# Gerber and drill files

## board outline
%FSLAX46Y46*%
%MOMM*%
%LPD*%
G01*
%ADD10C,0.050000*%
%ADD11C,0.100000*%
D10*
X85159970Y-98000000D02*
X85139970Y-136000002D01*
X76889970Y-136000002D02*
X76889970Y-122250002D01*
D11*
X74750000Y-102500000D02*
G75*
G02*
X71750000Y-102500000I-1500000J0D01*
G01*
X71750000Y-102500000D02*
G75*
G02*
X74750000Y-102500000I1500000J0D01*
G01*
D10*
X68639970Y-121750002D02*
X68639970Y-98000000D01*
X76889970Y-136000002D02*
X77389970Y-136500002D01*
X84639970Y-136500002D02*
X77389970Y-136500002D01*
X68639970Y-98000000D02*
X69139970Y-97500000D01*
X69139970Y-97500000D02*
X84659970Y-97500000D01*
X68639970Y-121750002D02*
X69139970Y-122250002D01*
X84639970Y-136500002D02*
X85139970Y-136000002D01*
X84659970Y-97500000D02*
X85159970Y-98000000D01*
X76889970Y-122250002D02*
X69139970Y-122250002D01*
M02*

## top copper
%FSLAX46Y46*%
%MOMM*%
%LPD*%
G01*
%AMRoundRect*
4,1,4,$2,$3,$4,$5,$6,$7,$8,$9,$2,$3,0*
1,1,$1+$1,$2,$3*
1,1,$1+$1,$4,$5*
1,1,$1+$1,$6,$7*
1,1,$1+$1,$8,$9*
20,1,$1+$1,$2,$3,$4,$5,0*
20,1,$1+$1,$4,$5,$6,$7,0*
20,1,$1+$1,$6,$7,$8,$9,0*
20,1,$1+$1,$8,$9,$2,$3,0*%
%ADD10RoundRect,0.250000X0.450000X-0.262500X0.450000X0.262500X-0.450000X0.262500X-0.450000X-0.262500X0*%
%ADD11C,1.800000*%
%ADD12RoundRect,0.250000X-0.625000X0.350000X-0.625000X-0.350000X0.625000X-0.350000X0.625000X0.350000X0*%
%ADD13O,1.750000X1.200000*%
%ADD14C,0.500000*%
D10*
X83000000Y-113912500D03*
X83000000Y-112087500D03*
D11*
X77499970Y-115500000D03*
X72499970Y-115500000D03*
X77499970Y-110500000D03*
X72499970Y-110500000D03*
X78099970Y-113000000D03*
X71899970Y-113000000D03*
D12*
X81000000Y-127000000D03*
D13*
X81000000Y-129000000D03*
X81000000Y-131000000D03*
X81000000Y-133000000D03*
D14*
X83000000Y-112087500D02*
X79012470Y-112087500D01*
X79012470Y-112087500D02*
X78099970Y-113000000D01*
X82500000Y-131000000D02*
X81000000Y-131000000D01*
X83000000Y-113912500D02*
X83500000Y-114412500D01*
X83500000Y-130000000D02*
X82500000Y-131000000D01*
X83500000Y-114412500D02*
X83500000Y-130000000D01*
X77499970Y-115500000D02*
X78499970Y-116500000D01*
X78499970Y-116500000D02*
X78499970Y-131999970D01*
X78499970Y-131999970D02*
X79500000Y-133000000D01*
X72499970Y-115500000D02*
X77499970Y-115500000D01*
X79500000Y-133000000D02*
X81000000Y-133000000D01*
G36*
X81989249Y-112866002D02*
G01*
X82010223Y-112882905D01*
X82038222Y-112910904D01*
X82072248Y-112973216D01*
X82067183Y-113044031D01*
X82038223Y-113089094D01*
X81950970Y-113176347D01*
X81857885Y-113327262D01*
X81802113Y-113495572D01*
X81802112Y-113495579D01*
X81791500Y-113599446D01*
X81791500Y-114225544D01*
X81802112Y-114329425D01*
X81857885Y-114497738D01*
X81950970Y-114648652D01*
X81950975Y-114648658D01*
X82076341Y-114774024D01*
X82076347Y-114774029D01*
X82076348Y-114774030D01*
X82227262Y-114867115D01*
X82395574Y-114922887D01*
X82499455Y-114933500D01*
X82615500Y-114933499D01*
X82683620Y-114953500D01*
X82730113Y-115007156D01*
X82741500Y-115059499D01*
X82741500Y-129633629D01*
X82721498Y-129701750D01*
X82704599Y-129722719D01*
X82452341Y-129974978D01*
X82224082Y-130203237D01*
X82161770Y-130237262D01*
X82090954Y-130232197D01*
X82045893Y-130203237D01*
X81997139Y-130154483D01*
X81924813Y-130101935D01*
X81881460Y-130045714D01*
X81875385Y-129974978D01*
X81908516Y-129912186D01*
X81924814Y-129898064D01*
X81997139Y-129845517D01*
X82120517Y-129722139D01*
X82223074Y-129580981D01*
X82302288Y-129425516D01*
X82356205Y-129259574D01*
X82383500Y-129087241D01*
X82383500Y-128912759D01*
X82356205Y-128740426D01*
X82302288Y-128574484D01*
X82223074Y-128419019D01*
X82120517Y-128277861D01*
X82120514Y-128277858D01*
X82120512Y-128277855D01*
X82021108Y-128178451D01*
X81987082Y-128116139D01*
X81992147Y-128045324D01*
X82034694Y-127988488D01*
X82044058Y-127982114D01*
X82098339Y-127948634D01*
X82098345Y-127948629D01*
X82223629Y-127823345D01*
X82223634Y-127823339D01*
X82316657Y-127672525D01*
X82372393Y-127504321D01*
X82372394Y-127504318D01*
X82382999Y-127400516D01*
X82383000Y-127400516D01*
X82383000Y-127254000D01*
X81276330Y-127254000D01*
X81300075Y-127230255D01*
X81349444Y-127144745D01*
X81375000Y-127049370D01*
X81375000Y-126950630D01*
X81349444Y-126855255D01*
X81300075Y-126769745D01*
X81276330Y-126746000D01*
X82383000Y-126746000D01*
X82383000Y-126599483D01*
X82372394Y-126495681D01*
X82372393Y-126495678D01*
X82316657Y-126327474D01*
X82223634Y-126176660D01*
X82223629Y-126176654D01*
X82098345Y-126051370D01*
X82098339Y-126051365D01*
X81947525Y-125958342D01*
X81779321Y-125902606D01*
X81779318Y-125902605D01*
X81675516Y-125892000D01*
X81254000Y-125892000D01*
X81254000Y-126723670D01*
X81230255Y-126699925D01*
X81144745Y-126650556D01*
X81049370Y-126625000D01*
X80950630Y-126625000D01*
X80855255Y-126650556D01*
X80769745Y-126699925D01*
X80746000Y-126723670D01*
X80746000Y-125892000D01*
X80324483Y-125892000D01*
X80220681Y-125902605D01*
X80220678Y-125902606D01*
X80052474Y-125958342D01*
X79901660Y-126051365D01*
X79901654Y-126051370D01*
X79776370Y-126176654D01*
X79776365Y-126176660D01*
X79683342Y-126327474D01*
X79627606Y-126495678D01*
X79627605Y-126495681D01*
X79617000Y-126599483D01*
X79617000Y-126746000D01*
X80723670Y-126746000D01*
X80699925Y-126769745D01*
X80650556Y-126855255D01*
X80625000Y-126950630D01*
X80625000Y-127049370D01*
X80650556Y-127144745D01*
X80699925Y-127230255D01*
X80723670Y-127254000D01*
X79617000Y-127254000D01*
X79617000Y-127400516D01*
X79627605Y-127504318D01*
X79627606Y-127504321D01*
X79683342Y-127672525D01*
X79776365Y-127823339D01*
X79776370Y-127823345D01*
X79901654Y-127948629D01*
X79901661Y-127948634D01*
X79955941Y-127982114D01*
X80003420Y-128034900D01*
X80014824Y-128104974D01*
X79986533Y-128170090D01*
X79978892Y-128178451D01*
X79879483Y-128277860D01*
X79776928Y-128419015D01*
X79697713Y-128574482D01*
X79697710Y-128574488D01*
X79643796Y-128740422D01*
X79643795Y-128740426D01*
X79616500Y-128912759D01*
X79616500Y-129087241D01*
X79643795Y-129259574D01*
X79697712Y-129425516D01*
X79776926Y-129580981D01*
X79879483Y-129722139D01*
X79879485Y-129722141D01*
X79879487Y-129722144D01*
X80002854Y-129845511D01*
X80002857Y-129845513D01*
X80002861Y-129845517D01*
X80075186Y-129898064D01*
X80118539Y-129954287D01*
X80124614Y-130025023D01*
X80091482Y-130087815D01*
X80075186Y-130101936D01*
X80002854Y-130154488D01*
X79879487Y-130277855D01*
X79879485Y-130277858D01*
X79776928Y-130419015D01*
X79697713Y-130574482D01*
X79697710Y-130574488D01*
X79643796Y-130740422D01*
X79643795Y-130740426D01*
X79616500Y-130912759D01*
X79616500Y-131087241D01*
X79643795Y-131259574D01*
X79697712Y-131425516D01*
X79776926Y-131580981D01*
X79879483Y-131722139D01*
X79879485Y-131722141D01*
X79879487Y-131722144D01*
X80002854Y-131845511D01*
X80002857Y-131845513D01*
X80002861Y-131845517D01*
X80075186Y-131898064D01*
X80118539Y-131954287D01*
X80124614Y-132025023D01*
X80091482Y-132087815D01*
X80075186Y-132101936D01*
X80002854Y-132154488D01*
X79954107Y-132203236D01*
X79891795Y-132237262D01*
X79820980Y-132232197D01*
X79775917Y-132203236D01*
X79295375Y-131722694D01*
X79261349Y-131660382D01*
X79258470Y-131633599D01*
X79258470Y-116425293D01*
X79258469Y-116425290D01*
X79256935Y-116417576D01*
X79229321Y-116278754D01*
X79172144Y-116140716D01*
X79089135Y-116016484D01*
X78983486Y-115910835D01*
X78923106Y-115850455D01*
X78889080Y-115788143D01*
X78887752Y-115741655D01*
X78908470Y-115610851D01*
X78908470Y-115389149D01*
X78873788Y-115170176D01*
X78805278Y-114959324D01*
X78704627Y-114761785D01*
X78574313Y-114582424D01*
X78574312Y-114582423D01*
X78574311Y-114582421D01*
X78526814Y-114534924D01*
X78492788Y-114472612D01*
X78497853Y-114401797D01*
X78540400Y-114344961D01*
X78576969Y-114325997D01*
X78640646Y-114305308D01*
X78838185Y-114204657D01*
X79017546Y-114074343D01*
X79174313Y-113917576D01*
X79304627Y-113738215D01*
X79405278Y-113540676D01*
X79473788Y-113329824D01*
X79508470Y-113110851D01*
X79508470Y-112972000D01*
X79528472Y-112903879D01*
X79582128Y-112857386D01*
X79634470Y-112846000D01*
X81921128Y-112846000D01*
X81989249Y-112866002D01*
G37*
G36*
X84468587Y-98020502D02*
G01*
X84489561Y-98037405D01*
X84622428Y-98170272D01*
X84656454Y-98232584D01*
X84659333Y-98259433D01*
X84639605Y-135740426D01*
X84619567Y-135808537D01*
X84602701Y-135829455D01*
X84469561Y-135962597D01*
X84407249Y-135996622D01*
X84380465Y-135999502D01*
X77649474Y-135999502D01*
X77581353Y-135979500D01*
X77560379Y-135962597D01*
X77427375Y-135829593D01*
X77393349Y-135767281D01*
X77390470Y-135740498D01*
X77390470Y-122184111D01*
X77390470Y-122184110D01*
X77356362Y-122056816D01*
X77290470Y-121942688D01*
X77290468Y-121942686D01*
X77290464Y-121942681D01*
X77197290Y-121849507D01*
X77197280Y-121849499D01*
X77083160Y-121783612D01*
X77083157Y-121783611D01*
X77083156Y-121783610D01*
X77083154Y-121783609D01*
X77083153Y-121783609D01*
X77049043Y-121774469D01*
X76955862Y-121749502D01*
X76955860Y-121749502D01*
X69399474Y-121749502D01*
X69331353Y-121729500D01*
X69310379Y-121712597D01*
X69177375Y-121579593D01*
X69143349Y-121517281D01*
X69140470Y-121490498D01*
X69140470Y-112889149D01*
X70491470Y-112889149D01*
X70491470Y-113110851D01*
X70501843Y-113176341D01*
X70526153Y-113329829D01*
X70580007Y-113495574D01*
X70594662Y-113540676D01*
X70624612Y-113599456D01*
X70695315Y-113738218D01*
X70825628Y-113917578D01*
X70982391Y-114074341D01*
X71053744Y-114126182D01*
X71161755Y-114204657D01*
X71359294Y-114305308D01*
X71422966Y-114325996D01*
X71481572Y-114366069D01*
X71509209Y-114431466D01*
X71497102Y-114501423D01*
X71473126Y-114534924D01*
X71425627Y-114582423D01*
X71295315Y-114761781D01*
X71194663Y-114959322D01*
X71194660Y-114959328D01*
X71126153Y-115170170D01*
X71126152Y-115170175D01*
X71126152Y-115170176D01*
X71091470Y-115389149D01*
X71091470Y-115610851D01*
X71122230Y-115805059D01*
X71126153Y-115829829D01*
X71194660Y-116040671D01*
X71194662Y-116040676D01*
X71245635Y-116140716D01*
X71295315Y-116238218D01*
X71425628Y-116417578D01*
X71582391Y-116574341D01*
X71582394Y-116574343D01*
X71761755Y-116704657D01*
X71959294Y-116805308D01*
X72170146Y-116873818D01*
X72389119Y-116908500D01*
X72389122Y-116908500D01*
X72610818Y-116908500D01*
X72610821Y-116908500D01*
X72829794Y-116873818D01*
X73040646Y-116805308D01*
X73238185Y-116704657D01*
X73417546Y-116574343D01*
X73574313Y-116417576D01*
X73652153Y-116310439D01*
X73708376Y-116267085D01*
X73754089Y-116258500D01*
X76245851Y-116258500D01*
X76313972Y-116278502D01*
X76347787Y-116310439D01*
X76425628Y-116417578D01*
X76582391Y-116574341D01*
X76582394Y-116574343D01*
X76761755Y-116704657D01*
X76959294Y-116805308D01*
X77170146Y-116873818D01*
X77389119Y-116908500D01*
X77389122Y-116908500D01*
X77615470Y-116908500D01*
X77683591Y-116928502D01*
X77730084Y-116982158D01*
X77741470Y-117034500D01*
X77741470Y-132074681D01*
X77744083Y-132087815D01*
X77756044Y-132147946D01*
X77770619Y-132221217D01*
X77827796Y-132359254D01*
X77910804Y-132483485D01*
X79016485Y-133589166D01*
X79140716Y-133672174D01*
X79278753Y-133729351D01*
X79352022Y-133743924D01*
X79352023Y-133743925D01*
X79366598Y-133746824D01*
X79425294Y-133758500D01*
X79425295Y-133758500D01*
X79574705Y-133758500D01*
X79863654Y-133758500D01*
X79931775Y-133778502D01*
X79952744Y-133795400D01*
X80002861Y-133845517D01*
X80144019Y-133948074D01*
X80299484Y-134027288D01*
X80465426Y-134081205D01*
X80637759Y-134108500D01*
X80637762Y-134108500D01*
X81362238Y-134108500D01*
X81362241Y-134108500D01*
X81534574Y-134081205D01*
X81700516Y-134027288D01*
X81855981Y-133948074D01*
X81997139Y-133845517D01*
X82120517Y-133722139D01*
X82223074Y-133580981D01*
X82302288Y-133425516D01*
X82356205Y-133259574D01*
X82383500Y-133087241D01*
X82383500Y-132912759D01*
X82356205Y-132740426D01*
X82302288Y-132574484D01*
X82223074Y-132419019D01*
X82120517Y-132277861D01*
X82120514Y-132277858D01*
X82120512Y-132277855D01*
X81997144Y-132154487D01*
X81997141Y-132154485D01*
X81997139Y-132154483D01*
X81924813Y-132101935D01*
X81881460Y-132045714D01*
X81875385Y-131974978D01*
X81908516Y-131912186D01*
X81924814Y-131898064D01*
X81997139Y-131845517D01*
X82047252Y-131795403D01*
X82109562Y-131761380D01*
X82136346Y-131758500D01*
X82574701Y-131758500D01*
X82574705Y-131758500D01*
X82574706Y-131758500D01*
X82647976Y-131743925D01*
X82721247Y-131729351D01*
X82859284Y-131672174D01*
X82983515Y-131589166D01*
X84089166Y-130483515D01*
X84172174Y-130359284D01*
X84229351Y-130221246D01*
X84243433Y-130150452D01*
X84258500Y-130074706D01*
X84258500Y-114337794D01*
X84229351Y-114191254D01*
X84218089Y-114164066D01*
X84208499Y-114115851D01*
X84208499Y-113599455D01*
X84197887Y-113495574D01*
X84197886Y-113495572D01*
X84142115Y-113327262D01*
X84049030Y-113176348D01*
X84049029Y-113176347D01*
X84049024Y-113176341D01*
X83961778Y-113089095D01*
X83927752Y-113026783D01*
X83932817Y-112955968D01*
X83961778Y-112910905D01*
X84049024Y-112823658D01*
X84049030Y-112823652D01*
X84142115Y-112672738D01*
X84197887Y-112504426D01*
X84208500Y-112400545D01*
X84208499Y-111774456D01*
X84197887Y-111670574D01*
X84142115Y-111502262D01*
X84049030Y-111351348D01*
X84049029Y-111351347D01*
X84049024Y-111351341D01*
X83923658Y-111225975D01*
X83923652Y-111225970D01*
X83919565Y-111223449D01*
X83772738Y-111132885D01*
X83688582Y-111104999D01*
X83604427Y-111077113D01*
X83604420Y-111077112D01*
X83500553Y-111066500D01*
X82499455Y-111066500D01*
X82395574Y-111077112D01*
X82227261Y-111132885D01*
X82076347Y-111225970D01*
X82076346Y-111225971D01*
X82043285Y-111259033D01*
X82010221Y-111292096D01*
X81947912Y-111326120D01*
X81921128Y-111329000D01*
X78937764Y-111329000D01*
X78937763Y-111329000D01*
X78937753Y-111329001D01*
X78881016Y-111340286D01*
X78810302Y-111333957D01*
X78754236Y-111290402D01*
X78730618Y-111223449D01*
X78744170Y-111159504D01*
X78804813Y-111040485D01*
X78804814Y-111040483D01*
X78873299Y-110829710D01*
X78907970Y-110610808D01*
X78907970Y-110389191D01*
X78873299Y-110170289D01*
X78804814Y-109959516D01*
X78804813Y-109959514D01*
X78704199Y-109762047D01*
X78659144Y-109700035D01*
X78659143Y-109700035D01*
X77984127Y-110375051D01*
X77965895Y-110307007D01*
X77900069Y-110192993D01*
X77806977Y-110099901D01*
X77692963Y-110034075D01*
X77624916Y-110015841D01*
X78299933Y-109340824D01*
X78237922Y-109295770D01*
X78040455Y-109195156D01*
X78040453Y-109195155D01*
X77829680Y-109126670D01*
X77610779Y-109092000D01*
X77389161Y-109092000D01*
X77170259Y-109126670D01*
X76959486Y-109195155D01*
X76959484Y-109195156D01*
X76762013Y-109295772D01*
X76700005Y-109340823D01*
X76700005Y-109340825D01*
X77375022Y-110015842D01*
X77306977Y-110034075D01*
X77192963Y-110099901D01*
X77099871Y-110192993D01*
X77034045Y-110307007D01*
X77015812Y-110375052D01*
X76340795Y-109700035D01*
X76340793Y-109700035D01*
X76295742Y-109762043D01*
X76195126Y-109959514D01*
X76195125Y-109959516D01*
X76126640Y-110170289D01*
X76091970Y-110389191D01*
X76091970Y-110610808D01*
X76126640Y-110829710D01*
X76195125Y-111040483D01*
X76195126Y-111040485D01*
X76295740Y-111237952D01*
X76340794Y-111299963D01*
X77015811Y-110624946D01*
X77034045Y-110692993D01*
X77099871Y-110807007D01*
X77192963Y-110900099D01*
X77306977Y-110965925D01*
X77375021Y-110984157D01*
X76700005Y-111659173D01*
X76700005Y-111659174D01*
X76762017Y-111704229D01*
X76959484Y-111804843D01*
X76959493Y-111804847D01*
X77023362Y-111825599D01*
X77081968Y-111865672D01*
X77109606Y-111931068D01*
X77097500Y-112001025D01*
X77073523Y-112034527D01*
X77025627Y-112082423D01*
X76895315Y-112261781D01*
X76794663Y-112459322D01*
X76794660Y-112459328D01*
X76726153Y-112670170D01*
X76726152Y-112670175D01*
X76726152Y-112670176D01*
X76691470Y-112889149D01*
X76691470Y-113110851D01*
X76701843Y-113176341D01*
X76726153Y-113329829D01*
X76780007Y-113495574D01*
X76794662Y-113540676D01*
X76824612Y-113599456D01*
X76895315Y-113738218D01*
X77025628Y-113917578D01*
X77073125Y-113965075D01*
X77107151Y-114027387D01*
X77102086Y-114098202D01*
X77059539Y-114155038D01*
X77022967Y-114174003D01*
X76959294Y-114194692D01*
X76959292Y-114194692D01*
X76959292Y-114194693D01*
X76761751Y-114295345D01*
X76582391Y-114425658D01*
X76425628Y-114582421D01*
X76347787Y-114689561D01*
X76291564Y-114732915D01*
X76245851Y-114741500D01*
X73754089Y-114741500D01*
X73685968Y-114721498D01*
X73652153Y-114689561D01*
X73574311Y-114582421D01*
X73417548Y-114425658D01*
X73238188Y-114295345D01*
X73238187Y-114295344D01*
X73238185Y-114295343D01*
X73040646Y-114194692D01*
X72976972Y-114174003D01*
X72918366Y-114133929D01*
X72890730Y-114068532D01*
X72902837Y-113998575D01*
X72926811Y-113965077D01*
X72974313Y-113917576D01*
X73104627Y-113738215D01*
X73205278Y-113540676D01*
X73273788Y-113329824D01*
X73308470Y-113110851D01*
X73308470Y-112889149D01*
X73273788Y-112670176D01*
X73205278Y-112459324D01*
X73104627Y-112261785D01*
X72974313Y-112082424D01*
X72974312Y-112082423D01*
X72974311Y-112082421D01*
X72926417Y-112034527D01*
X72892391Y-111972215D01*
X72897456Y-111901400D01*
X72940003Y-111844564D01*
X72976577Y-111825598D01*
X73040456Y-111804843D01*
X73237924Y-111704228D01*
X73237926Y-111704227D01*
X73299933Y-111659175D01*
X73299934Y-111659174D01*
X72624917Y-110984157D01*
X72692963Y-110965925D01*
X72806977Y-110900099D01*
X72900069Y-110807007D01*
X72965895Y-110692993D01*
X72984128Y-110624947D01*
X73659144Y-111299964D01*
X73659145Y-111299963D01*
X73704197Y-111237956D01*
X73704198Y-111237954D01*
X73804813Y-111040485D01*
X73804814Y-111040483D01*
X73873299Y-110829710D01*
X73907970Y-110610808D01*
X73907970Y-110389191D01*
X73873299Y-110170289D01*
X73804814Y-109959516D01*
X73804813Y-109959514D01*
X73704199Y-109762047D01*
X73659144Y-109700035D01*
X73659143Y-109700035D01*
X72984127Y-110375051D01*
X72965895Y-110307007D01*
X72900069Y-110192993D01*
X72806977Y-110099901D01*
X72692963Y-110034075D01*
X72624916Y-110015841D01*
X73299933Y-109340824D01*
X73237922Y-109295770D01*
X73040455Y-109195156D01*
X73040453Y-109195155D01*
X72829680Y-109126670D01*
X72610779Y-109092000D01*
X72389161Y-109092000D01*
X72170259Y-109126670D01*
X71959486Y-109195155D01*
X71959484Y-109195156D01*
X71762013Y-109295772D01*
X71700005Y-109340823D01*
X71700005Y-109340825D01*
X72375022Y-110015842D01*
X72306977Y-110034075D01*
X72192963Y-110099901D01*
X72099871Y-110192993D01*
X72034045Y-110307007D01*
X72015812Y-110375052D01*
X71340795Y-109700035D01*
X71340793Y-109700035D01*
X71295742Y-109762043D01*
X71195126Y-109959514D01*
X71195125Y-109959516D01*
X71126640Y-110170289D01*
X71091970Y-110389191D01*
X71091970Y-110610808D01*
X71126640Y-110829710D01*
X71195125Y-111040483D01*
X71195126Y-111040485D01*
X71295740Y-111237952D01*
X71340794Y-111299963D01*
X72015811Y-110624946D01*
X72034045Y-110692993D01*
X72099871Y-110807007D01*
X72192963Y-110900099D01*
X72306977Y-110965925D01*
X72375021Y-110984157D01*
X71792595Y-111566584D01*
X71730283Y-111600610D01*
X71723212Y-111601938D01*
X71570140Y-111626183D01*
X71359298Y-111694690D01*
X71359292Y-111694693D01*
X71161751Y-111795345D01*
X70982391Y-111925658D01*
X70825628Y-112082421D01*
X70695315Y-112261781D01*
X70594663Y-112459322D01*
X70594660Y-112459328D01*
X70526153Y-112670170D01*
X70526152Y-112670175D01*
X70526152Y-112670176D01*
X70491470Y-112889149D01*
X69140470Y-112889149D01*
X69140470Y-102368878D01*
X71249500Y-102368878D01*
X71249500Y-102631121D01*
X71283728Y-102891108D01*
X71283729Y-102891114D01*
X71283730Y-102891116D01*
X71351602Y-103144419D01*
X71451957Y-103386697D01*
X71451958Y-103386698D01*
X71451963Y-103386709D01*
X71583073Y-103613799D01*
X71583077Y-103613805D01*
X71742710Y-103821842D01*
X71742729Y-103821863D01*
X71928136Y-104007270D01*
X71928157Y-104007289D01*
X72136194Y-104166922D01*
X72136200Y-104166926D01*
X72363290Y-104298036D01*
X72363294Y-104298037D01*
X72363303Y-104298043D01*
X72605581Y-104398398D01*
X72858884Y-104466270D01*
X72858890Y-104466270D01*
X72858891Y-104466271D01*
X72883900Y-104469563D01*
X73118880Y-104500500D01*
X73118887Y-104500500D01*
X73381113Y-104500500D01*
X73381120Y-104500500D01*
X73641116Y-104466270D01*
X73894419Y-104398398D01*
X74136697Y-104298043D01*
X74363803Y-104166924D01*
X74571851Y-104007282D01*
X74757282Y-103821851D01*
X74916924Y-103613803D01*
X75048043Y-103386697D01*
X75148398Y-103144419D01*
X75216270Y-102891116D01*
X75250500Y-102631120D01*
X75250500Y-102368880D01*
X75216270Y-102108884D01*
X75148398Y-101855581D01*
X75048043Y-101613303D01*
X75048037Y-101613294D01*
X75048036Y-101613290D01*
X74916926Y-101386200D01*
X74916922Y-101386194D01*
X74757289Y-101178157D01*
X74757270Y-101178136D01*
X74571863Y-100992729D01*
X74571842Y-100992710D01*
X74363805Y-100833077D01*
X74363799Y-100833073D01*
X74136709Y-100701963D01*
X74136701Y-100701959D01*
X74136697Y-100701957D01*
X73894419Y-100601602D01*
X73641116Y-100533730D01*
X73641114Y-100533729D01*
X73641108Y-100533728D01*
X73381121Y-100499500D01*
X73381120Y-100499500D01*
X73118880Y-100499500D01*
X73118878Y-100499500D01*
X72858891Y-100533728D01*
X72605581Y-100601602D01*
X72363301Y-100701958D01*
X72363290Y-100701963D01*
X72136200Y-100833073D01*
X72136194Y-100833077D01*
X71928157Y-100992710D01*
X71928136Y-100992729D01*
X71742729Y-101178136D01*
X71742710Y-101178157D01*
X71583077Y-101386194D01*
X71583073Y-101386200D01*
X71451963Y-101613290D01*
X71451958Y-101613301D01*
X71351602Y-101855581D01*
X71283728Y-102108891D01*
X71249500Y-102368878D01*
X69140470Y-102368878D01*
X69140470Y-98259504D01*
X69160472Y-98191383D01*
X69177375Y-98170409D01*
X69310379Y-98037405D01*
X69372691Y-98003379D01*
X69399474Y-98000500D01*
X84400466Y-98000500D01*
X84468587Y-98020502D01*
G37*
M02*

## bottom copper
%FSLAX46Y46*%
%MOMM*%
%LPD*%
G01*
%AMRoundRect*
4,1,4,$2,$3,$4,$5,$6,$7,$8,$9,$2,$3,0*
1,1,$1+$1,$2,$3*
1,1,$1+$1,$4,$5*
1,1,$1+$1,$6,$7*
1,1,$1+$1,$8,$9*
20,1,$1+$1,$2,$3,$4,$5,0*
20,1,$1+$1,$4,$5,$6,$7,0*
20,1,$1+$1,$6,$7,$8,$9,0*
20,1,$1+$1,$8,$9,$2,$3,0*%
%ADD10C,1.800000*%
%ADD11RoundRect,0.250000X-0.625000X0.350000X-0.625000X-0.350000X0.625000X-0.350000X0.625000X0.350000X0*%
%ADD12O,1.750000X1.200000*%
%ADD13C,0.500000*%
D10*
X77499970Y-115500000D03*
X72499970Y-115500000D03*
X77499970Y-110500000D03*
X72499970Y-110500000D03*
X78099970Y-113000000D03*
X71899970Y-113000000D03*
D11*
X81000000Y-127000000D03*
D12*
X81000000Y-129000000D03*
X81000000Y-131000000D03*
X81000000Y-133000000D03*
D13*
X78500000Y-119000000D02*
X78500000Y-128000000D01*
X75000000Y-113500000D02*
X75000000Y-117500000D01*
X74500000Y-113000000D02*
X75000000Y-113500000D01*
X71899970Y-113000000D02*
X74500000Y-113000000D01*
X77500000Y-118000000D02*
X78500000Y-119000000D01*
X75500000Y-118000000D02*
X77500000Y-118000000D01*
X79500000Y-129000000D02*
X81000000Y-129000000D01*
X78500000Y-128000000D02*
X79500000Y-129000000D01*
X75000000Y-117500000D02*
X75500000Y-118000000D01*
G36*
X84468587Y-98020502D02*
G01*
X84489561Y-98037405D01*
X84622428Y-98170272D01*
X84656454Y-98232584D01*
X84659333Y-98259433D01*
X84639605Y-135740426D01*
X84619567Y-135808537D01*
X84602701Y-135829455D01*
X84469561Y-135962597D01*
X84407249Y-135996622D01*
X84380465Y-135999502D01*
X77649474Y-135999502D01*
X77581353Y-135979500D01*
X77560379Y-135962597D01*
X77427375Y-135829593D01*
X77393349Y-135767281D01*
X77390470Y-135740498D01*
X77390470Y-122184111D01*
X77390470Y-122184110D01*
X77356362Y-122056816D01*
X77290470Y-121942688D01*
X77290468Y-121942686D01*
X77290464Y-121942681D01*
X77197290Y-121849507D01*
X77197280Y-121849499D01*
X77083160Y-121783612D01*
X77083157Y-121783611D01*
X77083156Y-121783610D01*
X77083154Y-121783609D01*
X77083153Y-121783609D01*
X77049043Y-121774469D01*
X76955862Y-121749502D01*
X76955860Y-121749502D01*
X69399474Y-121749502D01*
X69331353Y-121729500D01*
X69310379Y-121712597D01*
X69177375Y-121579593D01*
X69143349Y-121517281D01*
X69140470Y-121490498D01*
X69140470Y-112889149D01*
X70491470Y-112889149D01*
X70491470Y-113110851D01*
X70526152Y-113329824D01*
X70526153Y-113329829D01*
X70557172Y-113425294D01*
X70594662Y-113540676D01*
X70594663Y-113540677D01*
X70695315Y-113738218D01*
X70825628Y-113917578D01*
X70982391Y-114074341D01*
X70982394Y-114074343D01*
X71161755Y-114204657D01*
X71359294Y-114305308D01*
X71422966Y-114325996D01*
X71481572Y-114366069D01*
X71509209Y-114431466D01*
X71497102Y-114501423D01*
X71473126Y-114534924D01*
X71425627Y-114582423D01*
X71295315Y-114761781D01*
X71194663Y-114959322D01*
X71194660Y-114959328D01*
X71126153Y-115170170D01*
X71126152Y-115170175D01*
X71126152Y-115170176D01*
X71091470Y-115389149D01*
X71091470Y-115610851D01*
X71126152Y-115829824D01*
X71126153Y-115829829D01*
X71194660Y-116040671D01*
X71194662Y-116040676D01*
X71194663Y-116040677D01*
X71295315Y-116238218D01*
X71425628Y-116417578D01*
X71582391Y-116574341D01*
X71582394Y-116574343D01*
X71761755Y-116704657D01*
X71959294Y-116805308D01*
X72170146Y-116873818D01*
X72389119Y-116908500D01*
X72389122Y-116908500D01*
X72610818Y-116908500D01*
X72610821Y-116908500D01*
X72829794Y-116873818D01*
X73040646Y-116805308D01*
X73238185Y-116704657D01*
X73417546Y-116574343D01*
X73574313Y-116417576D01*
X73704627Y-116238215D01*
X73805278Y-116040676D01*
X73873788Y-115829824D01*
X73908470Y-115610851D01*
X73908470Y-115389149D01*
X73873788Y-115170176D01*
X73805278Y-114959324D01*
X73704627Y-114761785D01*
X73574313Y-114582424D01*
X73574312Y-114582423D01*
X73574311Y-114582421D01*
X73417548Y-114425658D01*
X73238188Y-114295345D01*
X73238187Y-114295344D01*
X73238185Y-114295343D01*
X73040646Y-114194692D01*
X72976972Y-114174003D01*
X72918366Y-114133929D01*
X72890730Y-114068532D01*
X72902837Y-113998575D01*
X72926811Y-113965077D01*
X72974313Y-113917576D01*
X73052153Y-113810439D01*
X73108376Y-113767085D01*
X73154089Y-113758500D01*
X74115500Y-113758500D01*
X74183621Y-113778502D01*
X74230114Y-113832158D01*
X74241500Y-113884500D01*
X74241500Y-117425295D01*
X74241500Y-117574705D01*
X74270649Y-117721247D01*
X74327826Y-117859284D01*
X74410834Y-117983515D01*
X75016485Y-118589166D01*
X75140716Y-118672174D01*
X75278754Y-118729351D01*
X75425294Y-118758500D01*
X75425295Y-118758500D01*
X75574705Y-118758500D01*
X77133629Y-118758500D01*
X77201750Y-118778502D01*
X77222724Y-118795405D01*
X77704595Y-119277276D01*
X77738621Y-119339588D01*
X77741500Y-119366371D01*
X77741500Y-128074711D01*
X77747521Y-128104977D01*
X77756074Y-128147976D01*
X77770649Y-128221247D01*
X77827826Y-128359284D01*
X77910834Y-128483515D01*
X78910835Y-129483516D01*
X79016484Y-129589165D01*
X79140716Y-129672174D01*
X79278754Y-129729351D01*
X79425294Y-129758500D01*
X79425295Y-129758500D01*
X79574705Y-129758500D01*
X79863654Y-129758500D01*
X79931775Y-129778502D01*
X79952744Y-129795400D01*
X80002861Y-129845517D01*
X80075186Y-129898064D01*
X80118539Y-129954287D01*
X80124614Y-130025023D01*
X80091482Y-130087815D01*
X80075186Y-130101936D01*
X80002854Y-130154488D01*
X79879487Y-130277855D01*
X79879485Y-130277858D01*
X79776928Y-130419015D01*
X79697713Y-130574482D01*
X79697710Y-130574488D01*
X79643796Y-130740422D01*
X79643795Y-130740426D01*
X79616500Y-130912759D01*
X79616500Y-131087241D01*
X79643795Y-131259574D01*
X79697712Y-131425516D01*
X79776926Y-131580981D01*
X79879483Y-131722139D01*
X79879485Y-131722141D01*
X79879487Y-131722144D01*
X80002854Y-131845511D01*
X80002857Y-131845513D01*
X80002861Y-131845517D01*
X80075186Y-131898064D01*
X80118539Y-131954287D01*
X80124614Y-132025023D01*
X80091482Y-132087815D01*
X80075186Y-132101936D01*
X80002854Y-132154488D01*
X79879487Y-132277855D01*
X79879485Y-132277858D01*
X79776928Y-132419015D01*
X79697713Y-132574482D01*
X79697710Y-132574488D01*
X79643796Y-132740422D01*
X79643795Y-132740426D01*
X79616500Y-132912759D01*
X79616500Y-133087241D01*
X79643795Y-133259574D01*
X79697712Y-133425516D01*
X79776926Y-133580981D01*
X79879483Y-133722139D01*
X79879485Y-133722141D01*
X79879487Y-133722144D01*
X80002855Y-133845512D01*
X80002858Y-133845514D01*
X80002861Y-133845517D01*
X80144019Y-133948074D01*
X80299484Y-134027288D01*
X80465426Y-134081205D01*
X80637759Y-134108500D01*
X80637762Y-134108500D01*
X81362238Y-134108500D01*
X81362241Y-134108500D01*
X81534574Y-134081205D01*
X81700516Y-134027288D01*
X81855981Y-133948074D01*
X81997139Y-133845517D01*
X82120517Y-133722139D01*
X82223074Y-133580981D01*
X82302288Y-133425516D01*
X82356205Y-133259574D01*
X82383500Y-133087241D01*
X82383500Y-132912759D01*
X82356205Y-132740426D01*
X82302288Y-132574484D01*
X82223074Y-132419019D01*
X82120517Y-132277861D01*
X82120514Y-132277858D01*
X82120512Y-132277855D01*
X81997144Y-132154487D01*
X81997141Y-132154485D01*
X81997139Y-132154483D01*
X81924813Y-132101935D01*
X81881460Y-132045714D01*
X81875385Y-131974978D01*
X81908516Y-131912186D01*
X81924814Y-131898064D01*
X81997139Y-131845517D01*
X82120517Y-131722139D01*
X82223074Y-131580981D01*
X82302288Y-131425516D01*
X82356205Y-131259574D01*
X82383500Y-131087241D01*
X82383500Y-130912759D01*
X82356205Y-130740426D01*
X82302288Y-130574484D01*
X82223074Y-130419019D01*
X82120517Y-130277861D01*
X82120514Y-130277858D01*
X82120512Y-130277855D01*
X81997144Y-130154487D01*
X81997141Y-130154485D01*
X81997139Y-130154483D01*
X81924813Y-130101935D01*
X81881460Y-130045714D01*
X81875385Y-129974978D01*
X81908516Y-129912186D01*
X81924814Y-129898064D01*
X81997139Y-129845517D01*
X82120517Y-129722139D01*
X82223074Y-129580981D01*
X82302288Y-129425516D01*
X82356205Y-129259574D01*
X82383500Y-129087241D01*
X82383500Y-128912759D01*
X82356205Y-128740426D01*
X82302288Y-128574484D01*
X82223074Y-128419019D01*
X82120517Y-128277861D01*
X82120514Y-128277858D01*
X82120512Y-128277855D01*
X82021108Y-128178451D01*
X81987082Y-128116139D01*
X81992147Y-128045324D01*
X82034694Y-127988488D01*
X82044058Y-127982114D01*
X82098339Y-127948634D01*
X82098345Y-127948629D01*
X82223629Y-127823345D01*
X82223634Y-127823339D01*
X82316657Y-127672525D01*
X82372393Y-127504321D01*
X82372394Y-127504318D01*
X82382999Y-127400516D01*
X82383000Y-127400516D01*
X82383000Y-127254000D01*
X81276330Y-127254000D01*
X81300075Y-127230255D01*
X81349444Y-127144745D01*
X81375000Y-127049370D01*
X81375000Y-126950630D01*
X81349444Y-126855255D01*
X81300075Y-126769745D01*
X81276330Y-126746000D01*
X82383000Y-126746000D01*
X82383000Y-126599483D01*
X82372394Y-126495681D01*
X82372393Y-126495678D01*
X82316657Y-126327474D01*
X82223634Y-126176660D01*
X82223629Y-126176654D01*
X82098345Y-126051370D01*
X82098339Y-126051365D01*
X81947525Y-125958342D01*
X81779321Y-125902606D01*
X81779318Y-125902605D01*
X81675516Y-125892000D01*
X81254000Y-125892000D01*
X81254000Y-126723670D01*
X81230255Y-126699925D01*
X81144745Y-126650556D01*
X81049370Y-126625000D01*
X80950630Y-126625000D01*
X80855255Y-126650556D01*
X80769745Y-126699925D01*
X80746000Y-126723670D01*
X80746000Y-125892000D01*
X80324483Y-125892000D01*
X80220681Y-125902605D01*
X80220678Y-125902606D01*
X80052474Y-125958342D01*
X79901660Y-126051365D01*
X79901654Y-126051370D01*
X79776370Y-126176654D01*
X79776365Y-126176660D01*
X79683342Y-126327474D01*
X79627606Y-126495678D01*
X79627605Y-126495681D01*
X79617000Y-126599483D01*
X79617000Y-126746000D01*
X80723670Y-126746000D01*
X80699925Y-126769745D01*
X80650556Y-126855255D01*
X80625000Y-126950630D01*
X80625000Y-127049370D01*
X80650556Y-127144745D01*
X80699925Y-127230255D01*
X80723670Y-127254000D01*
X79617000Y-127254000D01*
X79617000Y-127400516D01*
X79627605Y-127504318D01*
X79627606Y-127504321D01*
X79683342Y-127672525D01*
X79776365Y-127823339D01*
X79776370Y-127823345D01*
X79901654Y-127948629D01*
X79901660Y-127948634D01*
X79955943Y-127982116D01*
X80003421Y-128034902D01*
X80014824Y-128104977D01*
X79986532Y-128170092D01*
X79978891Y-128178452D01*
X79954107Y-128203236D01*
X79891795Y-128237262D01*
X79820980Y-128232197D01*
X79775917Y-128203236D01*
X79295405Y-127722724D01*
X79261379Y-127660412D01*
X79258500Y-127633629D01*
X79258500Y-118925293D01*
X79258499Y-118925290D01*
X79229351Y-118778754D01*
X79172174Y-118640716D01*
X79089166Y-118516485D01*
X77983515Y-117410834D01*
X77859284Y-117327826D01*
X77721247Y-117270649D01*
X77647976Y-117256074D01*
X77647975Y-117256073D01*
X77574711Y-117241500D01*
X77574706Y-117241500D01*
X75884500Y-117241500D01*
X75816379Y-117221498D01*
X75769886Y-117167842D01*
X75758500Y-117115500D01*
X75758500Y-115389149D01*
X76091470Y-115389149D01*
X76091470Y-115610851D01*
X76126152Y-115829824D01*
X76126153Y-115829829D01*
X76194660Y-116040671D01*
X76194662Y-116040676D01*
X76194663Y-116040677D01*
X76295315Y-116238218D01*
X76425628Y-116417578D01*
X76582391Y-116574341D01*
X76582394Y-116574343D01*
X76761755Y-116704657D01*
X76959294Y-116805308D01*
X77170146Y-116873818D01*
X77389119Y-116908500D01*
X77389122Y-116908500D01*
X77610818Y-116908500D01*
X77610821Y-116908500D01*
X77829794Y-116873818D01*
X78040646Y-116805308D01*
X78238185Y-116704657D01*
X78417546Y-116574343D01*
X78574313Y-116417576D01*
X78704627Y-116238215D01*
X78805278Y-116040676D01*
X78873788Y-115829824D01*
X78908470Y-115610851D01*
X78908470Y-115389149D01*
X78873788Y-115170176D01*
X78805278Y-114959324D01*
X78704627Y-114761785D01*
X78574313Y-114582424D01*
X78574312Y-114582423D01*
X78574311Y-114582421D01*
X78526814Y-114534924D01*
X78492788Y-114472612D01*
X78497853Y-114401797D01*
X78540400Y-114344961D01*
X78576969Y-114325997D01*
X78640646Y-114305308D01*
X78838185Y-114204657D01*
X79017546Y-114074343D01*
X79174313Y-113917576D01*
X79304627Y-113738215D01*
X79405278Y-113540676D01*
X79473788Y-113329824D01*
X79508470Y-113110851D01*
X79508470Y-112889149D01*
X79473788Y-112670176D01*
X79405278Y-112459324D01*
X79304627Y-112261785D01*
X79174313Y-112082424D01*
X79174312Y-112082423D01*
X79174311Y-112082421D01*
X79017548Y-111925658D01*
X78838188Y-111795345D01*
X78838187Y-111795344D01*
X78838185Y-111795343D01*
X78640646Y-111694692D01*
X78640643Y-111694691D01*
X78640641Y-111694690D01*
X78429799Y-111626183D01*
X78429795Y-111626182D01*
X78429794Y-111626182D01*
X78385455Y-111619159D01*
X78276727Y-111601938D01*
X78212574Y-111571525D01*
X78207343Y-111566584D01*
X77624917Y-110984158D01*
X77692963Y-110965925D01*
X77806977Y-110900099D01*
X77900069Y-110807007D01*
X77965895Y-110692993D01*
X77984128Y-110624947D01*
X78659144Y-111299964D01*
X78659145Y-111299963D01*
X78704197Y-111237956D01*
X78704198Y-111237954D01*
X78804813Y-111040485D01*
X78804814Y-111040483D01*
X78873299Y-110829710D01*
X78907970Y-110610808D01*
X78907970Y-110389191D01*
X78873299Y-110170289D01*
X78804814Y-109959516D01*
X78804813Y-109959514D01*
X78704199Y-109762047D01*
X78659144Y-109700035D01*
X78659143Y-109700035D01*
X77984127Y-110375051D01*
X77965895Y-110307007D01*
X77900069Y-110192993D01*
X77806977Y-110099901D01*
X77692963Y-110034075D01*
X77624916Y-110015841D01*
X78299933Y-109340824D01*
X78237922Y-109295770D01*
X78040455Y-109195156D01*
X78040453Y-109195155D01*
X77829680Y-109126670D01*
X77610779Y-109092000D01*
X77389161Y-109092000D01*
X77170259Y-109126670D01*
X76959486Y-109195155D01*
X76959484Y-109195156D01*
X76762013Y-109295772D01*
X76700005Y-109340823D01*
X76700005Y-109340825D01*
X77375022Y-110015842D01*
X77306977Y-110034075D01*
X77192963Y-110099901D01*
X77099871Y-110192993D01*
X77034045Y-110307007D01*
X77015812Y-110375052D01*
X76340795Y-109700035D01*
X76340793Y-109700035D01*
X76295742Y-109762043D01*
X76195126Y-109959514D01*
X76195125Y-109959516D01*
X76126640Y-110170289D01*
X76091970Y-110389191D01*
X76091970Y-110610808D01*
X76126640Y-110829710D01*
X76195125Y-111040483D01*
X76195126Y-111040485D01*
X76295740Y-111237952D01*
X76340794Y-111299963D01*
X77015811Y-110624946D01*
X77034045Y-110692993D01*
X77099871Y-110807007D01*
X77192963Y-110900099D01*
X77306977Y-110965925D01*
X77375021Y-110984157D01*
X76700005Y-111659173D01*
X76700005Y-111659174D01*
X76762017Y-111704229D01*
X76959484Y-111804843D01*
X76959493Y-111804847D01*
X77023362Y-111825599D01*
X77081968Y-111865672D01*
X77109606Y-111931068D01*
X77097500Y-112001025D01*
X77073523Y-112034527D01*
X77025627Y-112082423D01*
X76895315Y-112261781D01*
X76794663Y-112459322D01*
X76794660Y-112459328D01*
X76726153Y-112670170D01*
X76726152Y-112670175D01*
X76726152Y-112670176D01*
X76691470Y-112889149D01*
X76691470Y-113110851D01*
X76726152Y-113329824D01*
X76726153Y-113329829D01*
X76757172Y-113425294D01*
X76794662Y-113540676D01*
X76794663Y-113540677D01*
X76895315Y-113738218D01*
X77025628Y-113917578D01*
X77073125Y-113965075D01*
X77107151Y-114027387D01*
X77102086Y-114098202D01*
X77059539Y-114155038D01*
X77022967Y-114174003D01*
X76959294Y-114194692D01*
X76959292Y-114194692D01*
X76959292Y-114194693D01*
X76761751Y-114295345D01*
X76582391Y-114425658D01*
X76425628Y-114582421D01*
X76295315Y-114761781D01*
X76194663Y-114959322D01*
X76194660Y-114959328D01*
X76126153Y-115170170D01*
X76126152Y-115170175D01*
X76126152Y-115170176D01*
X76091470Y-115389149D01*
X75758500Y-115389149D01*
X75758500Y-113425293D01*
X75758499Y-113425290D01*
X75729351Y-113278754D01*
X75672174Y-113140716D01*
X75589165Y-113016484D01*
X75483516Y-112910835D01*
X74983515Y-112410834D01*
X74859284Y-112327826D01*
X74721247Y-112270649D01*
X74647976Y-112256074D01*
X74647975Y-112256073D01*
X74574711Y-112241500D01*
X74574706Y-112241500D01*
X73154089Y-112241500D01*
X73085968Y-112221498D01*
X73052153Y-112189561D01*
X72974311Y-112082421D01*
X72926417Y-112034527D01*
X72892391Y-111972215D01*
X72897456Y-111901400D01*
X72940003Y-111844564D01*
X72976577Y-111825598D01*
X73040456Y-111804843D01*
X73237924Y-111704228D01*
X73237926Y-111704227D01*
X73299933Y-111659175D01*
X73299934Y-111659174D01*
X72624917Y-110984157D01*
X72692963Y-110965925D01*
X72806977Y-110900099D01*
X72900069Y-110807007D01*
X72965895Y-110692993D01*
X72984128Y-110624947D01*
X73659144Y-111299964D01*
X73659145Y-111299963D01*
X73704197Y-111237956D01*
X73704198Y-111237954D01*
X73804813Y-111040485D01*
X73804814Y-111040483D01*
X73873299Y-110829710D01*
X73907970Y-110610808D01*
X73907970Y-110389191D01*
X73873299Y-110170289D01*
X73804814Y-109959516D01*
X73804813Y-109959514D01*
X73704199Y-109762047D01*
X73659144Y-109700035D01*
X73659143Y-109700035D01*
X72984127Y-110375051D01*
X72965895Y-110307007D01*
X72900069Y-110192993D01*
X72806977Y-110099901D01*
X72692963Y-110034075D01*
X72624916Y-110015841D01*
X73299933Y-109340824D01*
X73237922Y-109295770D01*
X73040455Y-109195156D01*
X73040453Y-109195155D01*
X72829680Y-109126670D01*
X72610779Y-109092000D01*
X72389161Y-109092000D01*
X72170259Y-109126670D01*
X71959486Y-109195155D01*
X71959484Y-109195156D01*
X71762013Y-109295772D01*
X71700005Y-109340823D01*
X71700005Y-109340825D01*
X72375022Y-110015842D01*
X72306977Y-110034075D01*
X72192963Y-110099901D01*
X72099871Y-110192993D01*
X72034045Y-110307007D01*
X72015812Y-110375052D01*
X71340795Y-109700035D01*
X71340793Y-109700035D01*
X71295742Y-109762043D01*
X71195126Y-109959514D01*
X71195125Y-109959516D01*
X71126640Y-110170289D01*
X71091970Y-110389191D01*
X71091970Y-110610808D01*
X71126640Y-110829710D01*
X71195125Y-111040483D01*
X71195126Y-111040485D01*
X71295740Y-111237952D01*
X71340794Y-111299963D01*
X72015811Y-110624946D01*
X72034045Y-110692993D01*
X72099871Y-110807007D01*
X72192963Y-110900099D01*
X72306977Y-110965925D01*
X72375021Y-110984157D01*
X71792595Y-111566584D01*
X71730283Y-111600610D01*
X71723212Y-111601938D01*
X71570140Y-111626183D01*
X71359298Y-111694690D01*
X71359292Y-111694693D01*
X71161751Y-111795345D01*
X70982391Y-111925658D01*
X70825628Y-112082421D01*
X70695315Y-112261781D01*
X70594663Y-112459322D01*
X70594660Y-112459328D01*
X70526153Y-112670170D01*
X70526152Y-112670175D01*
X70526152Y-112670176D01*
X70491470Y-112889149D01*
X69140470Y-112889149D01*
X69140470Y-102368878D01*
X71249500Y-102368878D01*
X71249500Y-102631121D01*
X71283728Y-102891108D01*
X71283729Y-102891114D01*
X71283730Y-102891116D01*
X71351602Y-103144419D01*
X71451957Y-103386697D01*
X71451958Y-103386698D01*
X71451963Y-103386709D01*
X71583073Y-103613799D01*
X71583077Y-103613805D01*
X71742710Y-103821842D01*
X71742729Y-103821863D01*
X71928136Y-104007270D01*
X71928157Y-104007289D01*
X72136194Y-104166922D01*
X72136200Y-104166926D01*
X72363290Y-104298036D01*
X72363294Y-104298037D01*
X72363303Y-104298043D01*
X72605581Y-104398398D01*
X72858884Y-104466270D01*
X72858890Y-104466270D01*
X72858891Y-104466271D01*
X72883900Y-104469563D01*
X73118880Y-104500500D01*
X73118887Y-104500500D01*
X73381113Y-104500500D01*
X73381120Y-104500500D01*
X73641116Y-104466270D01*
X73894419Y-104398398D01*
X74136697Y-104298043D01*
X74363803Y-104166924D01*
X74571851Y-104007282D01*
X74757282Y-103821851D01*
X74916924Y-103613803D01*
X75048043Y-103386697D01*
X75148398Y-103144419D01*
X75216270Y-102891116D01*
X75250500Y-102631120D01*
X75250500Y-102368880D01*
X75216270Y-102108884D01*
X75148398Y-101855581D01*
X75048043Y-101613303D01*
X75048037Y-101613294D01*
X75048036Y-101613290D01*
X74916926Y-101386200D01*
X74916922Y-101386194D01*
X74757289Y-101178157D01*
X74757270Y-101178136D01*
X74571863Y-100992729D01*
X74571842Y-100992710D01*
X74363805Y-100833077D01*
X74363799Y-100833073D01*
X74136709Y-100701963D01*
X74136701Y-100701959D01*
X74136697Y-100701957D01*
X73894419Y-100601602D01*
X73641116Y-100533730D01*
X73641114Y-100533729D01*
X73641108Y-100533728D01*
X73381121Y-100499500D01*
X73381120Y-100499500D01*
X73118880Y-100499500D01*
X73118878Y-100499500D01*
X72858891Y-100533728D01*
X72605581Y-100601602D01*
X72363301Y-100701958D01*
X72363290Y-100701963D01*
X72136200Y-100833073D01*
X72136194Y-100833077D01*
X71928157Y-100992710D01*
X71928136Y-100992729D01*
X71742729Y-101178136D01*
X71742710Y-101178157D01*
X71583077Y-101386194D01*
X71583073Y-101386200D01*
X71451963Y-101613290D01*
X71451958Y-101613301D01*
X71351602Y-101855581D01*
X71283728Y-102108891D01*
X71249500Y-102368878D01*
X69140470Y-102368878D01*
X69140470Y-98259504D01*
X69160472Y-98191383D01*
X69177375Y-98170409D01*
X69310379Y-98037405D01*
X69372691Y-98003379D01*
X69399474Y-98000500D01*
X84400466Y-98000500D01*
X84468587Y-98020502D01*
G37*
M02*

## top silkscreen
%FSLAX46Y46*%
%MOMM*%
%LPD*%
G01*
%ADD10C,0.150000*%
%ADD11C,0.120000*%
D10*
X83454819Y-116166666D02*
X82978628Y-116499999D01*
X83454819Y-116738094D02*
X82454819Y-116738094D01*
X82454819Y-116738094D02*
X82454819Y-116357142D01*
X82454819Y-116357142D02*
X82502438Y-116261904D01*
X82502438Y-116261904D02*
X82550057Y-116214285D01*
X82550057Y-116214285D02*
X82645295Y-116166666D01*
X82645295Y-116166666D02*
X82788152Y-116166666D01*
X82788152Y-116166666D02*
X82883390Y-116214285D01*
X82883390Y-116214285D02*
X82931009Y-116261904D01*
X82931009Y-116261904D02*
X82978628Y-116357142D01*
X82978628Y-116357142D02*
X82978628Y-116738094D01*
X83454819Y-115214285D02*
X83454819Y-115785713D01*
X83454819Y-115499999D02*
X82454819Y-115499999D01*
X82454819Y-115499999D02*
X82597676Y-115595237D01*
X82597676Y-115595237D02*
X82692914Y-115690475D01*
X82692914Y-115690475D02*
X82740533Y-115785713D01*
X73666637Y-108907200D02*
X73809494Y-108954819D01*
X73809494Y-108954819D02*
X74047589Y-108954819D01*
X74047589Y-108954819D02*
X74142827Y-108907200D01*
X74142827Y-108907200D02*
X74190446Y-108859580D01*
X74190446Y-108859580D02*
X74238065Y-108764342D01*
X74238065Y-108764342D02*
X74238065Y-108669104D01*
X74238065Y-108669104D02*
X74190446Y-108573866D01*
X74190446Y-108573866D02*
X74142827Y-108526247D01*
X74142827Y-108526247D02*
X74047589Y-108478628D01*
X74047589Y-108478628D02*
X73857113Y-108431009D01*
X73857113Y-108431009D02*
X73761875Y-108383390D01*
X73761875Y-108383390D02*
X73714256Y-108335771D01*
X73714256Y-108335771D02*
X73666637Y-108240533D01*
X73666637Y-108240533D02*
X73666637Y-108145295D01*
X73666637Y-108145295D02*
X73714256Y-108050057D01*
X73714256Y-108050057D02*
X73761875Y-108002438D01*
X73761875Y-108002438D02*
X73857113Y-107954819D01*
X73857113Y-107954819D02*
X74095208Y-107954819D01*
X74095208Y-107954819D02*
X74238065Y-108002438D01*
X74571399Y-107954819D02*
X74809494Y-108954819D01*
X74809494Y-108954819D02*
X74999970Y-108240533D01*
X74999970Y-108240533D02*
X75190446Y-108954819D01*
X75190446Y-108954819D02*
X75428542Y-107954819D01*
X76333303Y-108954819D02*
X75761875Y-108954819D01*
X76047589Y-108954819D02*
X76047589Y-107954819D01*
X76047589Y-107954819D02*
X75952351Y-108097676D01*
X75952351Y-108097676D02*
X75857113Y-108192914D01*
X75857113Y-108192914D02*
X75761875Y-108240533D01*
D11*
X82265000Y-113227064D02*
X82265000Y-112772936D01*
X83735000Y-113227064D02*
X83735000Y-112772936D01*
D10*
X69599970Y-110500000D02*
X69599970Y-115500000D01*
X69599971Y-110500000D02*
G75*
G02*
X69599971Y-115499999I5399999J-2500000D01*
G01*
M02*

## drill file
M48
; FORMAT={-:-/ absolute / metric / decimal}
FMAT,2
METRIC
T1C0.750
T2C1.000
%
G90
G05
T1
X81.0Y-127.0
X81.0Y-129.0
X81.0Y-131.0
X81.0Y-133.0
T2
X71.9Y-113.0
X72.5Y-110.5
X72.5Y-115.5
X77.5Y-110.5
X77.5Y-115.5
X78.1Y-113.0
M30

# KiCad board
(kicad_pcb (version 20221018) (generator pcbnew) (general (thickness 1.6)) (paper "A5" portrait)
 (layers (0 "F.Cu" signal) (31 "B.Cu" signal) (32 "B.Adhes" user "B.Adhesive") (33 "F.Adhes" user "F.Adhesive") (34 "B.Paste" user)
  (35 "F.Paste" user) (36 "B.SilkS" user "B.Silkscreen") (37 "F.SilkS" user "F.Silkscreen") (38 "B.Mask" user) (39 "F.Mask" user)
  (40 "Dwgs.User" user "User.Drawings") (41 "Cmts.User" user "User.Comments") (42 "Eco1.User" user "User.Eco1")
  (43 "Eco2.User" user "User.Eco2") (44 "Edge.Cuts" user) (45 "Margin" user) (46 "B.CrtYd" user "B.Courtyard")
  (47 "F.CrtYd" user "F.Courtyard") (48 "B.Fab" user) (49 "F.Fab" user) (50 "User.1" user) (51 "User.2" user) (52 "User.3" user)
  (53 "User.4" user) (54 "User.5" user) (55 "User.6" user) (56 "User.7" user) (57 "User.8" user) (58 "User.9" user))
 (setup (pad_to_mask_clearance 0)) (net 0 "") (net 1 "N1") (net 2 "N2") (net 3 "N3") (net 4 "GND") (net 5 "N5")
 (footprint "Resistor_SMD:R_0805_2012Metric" (layer "F.Cu") (at 83 113 90)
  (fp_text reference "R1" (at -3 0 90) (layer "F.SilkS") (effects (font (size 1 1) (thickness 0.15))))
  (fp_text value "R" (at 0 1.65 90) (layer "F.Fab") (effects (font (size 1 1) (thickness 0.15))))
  (fp_line (start -0.227064 -0.735) (end 0.227064 -0.735) (stroke (width 0.12) (type solid)) (layer "F.SilkS"))
  (fp_line (start -0.227064 0.735) (end 0.227064 0.735) (stroke (width 0.12) (type solid)) (layer "F.SilkS"))
  (pad "1" smd roundrect (at -0.9125 0 90) (size 1.025 1.4) (layers "F.Cu" "F.Paste" "F.Mask") (roundrect_rratio 0.243902439) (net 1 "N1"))
  (pad "2" smd roundrect (at 0.9125 0 90) (size 1.025 1.4) (layers "F.Cu" "F.Paste" "F.Mask") (roundrect_rratio 0.243902439) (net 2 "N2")))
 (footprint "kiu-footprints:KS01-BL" (layer "F.Cu") (at 74.99997 113 180)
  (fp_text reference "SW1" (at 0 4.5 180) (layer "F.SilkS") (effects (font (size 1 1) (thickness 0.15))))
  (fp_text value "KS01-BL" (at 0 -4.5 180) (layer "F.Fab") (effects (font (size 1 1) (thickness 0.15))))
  (fp_line (start 5.4 2.5) (end 5.4 -2.5) (stroke (width 0.15) (type solid)) (layer "F.SilkS"))
  (fp_arc (start 5.399999 2.5) (mid -5.950629 0) (end 5.399999 -2.499999) (stroke (width 0.15) (type solid)) (layer "F.SilkS"))
  (pad "1" thru_hole circle (at -2.5 -2.5 180) (size 1.8 1.8) (drill 1) (layers "*.Cu" "*.Mask") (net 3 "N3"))
  (pad "1" thru_hole circle (at 2.5 -2.5 180) (size 1.8 1.8) (drill 1) (layers "*.Cu" "*.Mask") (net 3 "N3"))
  (pad "2" thru_hole circle (at -2.5 2.5 180) (size 1.8 1.8) (drill 1) (layers "*.Cu" "*.Mask") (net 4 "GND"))
  (pad "2" thru_hole circle (at 2.5 2.5 180) (size 1.8 1.8) (drill 1) (layers "*.Cu" "*.Mask") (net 4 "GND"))
  (pad "5" thru_hole circle (at -3.1 0 180) (size 1.8 1.8) (drill 1) (layers "*.Cu" "*.Mask") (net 2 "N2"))
  (pad "6" thru_hole circle (at 3.1 0 180) (size 1.8 1.8) (drill 1) (layers "*.Cu" "*.Mask") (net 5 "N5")))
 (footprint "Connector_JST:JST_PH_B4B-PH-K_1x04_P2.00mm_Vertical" (layer "B.Cu") (at 81 127 -90)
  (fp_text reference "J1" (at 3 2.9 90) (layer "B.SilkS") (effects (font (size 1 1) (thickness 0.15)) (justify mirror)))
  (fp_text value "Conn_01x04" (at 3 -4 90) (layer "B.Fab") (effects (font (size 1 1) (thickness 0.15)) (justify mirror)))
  (pad "1" thru_hole roundrect (at 0 0 270) (size 1.2 1.75) (drill 0.75) (layers "*.Cu" "*.Mask") (roundrect_rratio 0.2083333333)
   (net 4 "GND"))
  (pad "2" thru_hole oval (at 2 0 270) (size 1.2 1.75) (drill 0.75) (layers "*.Cu" "*.Mask") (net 5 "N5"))
  (pad "3" thru_hole oval (at 4 0 270) (size 1.2 1.75) (drill 0.75) (layers "*.Cu" "*.Mask") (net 1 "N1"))
  (pad "4" thru_hole oval (at 6 0 270) (size 1.2 1.75) (drill 0.75) (layers "*.Cu" "*.Mask") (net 3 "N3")))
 (gr_line (start 85.15997 98) (end 85.13997 136.000002) (stroke (width 0.05) (type solid)) (layer "Edge.Cuts"))
 (gr_line (start 76.88997 136.000002) (end 76.88997 122.250002) (stroke (width 0.05) (type default)) (layer "Edge.Cuts"))
 (gr_circle (center 73.25 102.5) (end 74.75 102.5) (stroke (width 0.1) (type default)) (fill none) (layer "Edge.Cuts"))
 (gr_line (start 68.63997 121.750002) (end 68.63997 98) (stroke (width 0.05) (type default)) (layer "Edge.Cuts"))
 (gr_line (start 76.88997 136.000002) (end 77.38997 136.500002) (stroke (width 0.05) (type default)) (layer "Edge.Cuts"))
 (gr_line (start 84.63997 136.500002) (end 77.38997 136.500002) (stroke (width 0.05) (type solid)) (layer "Edge.Cuts"))
 (gr_line (start 68.63997 98) (end 69.13997 97.5) (stroke (width 0.05) (type default)) (layer "Edge.Cuts"))
 (gr_line (start 69.13997 97.5) (end 84.65997 97.5) (stroke (width 0.05) (type default)) (layer "Edge.Cuts"))
 (gr_line (start 68.63997 121.750002) (end 69.13997 122.250002) (stroke (width 0.05) (type default)) (layer "Edge.Cuts"))
 (gr_line (start 84.63997 136.500002) (end 85.13997 136.000002) (stroke (width 0.05) (type default)) (layer "Edge.Cuts"))
 (gr_line (start 84.65997 97.5) (end 85.15997 98) (stroke (width 0.05) (type default)) (layer "Edge.Cuts"))
 (gr_line (start 76.88997 122.250002) (end 69.13997 122.250002) (stroke (width 0.05) (type default)) (layer "Edge.Cuts"))
 (segment (start 83 112.0875) (end 79.01247 112.0875) (width 0.5) (layer "F.Cu") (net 2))
 (segment (start 79.01247 112.0875) (end 78.09997 113) (width 0.5) (layer "F.Cu") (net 2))
 (segment (start 82.5 131) (end 81 131) (width 0.5) (layer "F.Cu") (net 1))
 (segment (start 83 113.9125) (end 83.5 114.4125) (width 0.5) (layer "F.Cu") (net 1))
 (segment (start 83.5 130) (end 82.5 131) (width 0.5) (layer "F.Cu") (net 1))
 (segment (start 83.5 114.4125) (end 83.5 130) (width 0.5) (layer "F.Cu") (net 1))
 (segment (start 77.49997 115.5) (end 78.49997 116.5) (width 0.5) (layer "F.Cu") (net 3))
 (segment (start 78.49997 116.5) (end 78.49997 131.99997) (width 0.5) (layer "F.Cu") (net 3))
 (segment (start 78.49997 131.99997) (end 79.5 133) (width 0.5) (layer "F.Cu") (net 3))
 (segment (start 72.49997 115.5) (end 77.49997 115.5) (width 0.5) (layer "F.Cu") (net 3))
 (segment (start 79.5 133) (end 81 133) (width 0.5) (layer "F.Cu") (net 3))
 (segment (start 78.5 119) (end 78.5 128) (width 0.5) (layer "B.Cu") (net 5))
 (segment (start 75 113.5) (end 75 117.5) (width 0.5) (layer "B.Cu") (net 5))
 (segment (start 74.5 113) (end 75 113.5) (width 0.5) (layer "B.Cu") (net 5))
 (segment (start 71.89997 113) (end 74.5 113) (width 0.5) (layer "B.Cu") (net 5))
 (segment (start 77.5 118) (end 78.5 119) (width 0.5) (layer "B.Cu") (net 5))
 (segment (start 75.5 118) (end 77.5 118) (width 0.5) (layer "B.Cu") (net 5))
 (segment (start 79.5 129) (end 81 129) (width 0.5) (layer "B.Cu") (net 5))
 (segment (start 78.5 128) (end 79.5 129) (width 0.5) (layer "B.Cu") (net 5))
 (segment (start 75 117.5) (end 75.5 118) (width 0.5) (layer "B.Cu") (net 5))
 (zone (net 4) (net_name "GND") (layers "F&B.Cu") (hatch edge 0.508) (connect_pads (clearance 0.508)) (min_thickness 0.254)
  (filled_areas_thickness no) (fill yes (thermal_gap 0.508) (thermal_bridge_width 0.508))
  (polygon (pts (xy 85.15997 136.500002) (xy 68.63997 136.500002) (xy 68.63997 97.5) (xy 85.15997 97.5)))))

